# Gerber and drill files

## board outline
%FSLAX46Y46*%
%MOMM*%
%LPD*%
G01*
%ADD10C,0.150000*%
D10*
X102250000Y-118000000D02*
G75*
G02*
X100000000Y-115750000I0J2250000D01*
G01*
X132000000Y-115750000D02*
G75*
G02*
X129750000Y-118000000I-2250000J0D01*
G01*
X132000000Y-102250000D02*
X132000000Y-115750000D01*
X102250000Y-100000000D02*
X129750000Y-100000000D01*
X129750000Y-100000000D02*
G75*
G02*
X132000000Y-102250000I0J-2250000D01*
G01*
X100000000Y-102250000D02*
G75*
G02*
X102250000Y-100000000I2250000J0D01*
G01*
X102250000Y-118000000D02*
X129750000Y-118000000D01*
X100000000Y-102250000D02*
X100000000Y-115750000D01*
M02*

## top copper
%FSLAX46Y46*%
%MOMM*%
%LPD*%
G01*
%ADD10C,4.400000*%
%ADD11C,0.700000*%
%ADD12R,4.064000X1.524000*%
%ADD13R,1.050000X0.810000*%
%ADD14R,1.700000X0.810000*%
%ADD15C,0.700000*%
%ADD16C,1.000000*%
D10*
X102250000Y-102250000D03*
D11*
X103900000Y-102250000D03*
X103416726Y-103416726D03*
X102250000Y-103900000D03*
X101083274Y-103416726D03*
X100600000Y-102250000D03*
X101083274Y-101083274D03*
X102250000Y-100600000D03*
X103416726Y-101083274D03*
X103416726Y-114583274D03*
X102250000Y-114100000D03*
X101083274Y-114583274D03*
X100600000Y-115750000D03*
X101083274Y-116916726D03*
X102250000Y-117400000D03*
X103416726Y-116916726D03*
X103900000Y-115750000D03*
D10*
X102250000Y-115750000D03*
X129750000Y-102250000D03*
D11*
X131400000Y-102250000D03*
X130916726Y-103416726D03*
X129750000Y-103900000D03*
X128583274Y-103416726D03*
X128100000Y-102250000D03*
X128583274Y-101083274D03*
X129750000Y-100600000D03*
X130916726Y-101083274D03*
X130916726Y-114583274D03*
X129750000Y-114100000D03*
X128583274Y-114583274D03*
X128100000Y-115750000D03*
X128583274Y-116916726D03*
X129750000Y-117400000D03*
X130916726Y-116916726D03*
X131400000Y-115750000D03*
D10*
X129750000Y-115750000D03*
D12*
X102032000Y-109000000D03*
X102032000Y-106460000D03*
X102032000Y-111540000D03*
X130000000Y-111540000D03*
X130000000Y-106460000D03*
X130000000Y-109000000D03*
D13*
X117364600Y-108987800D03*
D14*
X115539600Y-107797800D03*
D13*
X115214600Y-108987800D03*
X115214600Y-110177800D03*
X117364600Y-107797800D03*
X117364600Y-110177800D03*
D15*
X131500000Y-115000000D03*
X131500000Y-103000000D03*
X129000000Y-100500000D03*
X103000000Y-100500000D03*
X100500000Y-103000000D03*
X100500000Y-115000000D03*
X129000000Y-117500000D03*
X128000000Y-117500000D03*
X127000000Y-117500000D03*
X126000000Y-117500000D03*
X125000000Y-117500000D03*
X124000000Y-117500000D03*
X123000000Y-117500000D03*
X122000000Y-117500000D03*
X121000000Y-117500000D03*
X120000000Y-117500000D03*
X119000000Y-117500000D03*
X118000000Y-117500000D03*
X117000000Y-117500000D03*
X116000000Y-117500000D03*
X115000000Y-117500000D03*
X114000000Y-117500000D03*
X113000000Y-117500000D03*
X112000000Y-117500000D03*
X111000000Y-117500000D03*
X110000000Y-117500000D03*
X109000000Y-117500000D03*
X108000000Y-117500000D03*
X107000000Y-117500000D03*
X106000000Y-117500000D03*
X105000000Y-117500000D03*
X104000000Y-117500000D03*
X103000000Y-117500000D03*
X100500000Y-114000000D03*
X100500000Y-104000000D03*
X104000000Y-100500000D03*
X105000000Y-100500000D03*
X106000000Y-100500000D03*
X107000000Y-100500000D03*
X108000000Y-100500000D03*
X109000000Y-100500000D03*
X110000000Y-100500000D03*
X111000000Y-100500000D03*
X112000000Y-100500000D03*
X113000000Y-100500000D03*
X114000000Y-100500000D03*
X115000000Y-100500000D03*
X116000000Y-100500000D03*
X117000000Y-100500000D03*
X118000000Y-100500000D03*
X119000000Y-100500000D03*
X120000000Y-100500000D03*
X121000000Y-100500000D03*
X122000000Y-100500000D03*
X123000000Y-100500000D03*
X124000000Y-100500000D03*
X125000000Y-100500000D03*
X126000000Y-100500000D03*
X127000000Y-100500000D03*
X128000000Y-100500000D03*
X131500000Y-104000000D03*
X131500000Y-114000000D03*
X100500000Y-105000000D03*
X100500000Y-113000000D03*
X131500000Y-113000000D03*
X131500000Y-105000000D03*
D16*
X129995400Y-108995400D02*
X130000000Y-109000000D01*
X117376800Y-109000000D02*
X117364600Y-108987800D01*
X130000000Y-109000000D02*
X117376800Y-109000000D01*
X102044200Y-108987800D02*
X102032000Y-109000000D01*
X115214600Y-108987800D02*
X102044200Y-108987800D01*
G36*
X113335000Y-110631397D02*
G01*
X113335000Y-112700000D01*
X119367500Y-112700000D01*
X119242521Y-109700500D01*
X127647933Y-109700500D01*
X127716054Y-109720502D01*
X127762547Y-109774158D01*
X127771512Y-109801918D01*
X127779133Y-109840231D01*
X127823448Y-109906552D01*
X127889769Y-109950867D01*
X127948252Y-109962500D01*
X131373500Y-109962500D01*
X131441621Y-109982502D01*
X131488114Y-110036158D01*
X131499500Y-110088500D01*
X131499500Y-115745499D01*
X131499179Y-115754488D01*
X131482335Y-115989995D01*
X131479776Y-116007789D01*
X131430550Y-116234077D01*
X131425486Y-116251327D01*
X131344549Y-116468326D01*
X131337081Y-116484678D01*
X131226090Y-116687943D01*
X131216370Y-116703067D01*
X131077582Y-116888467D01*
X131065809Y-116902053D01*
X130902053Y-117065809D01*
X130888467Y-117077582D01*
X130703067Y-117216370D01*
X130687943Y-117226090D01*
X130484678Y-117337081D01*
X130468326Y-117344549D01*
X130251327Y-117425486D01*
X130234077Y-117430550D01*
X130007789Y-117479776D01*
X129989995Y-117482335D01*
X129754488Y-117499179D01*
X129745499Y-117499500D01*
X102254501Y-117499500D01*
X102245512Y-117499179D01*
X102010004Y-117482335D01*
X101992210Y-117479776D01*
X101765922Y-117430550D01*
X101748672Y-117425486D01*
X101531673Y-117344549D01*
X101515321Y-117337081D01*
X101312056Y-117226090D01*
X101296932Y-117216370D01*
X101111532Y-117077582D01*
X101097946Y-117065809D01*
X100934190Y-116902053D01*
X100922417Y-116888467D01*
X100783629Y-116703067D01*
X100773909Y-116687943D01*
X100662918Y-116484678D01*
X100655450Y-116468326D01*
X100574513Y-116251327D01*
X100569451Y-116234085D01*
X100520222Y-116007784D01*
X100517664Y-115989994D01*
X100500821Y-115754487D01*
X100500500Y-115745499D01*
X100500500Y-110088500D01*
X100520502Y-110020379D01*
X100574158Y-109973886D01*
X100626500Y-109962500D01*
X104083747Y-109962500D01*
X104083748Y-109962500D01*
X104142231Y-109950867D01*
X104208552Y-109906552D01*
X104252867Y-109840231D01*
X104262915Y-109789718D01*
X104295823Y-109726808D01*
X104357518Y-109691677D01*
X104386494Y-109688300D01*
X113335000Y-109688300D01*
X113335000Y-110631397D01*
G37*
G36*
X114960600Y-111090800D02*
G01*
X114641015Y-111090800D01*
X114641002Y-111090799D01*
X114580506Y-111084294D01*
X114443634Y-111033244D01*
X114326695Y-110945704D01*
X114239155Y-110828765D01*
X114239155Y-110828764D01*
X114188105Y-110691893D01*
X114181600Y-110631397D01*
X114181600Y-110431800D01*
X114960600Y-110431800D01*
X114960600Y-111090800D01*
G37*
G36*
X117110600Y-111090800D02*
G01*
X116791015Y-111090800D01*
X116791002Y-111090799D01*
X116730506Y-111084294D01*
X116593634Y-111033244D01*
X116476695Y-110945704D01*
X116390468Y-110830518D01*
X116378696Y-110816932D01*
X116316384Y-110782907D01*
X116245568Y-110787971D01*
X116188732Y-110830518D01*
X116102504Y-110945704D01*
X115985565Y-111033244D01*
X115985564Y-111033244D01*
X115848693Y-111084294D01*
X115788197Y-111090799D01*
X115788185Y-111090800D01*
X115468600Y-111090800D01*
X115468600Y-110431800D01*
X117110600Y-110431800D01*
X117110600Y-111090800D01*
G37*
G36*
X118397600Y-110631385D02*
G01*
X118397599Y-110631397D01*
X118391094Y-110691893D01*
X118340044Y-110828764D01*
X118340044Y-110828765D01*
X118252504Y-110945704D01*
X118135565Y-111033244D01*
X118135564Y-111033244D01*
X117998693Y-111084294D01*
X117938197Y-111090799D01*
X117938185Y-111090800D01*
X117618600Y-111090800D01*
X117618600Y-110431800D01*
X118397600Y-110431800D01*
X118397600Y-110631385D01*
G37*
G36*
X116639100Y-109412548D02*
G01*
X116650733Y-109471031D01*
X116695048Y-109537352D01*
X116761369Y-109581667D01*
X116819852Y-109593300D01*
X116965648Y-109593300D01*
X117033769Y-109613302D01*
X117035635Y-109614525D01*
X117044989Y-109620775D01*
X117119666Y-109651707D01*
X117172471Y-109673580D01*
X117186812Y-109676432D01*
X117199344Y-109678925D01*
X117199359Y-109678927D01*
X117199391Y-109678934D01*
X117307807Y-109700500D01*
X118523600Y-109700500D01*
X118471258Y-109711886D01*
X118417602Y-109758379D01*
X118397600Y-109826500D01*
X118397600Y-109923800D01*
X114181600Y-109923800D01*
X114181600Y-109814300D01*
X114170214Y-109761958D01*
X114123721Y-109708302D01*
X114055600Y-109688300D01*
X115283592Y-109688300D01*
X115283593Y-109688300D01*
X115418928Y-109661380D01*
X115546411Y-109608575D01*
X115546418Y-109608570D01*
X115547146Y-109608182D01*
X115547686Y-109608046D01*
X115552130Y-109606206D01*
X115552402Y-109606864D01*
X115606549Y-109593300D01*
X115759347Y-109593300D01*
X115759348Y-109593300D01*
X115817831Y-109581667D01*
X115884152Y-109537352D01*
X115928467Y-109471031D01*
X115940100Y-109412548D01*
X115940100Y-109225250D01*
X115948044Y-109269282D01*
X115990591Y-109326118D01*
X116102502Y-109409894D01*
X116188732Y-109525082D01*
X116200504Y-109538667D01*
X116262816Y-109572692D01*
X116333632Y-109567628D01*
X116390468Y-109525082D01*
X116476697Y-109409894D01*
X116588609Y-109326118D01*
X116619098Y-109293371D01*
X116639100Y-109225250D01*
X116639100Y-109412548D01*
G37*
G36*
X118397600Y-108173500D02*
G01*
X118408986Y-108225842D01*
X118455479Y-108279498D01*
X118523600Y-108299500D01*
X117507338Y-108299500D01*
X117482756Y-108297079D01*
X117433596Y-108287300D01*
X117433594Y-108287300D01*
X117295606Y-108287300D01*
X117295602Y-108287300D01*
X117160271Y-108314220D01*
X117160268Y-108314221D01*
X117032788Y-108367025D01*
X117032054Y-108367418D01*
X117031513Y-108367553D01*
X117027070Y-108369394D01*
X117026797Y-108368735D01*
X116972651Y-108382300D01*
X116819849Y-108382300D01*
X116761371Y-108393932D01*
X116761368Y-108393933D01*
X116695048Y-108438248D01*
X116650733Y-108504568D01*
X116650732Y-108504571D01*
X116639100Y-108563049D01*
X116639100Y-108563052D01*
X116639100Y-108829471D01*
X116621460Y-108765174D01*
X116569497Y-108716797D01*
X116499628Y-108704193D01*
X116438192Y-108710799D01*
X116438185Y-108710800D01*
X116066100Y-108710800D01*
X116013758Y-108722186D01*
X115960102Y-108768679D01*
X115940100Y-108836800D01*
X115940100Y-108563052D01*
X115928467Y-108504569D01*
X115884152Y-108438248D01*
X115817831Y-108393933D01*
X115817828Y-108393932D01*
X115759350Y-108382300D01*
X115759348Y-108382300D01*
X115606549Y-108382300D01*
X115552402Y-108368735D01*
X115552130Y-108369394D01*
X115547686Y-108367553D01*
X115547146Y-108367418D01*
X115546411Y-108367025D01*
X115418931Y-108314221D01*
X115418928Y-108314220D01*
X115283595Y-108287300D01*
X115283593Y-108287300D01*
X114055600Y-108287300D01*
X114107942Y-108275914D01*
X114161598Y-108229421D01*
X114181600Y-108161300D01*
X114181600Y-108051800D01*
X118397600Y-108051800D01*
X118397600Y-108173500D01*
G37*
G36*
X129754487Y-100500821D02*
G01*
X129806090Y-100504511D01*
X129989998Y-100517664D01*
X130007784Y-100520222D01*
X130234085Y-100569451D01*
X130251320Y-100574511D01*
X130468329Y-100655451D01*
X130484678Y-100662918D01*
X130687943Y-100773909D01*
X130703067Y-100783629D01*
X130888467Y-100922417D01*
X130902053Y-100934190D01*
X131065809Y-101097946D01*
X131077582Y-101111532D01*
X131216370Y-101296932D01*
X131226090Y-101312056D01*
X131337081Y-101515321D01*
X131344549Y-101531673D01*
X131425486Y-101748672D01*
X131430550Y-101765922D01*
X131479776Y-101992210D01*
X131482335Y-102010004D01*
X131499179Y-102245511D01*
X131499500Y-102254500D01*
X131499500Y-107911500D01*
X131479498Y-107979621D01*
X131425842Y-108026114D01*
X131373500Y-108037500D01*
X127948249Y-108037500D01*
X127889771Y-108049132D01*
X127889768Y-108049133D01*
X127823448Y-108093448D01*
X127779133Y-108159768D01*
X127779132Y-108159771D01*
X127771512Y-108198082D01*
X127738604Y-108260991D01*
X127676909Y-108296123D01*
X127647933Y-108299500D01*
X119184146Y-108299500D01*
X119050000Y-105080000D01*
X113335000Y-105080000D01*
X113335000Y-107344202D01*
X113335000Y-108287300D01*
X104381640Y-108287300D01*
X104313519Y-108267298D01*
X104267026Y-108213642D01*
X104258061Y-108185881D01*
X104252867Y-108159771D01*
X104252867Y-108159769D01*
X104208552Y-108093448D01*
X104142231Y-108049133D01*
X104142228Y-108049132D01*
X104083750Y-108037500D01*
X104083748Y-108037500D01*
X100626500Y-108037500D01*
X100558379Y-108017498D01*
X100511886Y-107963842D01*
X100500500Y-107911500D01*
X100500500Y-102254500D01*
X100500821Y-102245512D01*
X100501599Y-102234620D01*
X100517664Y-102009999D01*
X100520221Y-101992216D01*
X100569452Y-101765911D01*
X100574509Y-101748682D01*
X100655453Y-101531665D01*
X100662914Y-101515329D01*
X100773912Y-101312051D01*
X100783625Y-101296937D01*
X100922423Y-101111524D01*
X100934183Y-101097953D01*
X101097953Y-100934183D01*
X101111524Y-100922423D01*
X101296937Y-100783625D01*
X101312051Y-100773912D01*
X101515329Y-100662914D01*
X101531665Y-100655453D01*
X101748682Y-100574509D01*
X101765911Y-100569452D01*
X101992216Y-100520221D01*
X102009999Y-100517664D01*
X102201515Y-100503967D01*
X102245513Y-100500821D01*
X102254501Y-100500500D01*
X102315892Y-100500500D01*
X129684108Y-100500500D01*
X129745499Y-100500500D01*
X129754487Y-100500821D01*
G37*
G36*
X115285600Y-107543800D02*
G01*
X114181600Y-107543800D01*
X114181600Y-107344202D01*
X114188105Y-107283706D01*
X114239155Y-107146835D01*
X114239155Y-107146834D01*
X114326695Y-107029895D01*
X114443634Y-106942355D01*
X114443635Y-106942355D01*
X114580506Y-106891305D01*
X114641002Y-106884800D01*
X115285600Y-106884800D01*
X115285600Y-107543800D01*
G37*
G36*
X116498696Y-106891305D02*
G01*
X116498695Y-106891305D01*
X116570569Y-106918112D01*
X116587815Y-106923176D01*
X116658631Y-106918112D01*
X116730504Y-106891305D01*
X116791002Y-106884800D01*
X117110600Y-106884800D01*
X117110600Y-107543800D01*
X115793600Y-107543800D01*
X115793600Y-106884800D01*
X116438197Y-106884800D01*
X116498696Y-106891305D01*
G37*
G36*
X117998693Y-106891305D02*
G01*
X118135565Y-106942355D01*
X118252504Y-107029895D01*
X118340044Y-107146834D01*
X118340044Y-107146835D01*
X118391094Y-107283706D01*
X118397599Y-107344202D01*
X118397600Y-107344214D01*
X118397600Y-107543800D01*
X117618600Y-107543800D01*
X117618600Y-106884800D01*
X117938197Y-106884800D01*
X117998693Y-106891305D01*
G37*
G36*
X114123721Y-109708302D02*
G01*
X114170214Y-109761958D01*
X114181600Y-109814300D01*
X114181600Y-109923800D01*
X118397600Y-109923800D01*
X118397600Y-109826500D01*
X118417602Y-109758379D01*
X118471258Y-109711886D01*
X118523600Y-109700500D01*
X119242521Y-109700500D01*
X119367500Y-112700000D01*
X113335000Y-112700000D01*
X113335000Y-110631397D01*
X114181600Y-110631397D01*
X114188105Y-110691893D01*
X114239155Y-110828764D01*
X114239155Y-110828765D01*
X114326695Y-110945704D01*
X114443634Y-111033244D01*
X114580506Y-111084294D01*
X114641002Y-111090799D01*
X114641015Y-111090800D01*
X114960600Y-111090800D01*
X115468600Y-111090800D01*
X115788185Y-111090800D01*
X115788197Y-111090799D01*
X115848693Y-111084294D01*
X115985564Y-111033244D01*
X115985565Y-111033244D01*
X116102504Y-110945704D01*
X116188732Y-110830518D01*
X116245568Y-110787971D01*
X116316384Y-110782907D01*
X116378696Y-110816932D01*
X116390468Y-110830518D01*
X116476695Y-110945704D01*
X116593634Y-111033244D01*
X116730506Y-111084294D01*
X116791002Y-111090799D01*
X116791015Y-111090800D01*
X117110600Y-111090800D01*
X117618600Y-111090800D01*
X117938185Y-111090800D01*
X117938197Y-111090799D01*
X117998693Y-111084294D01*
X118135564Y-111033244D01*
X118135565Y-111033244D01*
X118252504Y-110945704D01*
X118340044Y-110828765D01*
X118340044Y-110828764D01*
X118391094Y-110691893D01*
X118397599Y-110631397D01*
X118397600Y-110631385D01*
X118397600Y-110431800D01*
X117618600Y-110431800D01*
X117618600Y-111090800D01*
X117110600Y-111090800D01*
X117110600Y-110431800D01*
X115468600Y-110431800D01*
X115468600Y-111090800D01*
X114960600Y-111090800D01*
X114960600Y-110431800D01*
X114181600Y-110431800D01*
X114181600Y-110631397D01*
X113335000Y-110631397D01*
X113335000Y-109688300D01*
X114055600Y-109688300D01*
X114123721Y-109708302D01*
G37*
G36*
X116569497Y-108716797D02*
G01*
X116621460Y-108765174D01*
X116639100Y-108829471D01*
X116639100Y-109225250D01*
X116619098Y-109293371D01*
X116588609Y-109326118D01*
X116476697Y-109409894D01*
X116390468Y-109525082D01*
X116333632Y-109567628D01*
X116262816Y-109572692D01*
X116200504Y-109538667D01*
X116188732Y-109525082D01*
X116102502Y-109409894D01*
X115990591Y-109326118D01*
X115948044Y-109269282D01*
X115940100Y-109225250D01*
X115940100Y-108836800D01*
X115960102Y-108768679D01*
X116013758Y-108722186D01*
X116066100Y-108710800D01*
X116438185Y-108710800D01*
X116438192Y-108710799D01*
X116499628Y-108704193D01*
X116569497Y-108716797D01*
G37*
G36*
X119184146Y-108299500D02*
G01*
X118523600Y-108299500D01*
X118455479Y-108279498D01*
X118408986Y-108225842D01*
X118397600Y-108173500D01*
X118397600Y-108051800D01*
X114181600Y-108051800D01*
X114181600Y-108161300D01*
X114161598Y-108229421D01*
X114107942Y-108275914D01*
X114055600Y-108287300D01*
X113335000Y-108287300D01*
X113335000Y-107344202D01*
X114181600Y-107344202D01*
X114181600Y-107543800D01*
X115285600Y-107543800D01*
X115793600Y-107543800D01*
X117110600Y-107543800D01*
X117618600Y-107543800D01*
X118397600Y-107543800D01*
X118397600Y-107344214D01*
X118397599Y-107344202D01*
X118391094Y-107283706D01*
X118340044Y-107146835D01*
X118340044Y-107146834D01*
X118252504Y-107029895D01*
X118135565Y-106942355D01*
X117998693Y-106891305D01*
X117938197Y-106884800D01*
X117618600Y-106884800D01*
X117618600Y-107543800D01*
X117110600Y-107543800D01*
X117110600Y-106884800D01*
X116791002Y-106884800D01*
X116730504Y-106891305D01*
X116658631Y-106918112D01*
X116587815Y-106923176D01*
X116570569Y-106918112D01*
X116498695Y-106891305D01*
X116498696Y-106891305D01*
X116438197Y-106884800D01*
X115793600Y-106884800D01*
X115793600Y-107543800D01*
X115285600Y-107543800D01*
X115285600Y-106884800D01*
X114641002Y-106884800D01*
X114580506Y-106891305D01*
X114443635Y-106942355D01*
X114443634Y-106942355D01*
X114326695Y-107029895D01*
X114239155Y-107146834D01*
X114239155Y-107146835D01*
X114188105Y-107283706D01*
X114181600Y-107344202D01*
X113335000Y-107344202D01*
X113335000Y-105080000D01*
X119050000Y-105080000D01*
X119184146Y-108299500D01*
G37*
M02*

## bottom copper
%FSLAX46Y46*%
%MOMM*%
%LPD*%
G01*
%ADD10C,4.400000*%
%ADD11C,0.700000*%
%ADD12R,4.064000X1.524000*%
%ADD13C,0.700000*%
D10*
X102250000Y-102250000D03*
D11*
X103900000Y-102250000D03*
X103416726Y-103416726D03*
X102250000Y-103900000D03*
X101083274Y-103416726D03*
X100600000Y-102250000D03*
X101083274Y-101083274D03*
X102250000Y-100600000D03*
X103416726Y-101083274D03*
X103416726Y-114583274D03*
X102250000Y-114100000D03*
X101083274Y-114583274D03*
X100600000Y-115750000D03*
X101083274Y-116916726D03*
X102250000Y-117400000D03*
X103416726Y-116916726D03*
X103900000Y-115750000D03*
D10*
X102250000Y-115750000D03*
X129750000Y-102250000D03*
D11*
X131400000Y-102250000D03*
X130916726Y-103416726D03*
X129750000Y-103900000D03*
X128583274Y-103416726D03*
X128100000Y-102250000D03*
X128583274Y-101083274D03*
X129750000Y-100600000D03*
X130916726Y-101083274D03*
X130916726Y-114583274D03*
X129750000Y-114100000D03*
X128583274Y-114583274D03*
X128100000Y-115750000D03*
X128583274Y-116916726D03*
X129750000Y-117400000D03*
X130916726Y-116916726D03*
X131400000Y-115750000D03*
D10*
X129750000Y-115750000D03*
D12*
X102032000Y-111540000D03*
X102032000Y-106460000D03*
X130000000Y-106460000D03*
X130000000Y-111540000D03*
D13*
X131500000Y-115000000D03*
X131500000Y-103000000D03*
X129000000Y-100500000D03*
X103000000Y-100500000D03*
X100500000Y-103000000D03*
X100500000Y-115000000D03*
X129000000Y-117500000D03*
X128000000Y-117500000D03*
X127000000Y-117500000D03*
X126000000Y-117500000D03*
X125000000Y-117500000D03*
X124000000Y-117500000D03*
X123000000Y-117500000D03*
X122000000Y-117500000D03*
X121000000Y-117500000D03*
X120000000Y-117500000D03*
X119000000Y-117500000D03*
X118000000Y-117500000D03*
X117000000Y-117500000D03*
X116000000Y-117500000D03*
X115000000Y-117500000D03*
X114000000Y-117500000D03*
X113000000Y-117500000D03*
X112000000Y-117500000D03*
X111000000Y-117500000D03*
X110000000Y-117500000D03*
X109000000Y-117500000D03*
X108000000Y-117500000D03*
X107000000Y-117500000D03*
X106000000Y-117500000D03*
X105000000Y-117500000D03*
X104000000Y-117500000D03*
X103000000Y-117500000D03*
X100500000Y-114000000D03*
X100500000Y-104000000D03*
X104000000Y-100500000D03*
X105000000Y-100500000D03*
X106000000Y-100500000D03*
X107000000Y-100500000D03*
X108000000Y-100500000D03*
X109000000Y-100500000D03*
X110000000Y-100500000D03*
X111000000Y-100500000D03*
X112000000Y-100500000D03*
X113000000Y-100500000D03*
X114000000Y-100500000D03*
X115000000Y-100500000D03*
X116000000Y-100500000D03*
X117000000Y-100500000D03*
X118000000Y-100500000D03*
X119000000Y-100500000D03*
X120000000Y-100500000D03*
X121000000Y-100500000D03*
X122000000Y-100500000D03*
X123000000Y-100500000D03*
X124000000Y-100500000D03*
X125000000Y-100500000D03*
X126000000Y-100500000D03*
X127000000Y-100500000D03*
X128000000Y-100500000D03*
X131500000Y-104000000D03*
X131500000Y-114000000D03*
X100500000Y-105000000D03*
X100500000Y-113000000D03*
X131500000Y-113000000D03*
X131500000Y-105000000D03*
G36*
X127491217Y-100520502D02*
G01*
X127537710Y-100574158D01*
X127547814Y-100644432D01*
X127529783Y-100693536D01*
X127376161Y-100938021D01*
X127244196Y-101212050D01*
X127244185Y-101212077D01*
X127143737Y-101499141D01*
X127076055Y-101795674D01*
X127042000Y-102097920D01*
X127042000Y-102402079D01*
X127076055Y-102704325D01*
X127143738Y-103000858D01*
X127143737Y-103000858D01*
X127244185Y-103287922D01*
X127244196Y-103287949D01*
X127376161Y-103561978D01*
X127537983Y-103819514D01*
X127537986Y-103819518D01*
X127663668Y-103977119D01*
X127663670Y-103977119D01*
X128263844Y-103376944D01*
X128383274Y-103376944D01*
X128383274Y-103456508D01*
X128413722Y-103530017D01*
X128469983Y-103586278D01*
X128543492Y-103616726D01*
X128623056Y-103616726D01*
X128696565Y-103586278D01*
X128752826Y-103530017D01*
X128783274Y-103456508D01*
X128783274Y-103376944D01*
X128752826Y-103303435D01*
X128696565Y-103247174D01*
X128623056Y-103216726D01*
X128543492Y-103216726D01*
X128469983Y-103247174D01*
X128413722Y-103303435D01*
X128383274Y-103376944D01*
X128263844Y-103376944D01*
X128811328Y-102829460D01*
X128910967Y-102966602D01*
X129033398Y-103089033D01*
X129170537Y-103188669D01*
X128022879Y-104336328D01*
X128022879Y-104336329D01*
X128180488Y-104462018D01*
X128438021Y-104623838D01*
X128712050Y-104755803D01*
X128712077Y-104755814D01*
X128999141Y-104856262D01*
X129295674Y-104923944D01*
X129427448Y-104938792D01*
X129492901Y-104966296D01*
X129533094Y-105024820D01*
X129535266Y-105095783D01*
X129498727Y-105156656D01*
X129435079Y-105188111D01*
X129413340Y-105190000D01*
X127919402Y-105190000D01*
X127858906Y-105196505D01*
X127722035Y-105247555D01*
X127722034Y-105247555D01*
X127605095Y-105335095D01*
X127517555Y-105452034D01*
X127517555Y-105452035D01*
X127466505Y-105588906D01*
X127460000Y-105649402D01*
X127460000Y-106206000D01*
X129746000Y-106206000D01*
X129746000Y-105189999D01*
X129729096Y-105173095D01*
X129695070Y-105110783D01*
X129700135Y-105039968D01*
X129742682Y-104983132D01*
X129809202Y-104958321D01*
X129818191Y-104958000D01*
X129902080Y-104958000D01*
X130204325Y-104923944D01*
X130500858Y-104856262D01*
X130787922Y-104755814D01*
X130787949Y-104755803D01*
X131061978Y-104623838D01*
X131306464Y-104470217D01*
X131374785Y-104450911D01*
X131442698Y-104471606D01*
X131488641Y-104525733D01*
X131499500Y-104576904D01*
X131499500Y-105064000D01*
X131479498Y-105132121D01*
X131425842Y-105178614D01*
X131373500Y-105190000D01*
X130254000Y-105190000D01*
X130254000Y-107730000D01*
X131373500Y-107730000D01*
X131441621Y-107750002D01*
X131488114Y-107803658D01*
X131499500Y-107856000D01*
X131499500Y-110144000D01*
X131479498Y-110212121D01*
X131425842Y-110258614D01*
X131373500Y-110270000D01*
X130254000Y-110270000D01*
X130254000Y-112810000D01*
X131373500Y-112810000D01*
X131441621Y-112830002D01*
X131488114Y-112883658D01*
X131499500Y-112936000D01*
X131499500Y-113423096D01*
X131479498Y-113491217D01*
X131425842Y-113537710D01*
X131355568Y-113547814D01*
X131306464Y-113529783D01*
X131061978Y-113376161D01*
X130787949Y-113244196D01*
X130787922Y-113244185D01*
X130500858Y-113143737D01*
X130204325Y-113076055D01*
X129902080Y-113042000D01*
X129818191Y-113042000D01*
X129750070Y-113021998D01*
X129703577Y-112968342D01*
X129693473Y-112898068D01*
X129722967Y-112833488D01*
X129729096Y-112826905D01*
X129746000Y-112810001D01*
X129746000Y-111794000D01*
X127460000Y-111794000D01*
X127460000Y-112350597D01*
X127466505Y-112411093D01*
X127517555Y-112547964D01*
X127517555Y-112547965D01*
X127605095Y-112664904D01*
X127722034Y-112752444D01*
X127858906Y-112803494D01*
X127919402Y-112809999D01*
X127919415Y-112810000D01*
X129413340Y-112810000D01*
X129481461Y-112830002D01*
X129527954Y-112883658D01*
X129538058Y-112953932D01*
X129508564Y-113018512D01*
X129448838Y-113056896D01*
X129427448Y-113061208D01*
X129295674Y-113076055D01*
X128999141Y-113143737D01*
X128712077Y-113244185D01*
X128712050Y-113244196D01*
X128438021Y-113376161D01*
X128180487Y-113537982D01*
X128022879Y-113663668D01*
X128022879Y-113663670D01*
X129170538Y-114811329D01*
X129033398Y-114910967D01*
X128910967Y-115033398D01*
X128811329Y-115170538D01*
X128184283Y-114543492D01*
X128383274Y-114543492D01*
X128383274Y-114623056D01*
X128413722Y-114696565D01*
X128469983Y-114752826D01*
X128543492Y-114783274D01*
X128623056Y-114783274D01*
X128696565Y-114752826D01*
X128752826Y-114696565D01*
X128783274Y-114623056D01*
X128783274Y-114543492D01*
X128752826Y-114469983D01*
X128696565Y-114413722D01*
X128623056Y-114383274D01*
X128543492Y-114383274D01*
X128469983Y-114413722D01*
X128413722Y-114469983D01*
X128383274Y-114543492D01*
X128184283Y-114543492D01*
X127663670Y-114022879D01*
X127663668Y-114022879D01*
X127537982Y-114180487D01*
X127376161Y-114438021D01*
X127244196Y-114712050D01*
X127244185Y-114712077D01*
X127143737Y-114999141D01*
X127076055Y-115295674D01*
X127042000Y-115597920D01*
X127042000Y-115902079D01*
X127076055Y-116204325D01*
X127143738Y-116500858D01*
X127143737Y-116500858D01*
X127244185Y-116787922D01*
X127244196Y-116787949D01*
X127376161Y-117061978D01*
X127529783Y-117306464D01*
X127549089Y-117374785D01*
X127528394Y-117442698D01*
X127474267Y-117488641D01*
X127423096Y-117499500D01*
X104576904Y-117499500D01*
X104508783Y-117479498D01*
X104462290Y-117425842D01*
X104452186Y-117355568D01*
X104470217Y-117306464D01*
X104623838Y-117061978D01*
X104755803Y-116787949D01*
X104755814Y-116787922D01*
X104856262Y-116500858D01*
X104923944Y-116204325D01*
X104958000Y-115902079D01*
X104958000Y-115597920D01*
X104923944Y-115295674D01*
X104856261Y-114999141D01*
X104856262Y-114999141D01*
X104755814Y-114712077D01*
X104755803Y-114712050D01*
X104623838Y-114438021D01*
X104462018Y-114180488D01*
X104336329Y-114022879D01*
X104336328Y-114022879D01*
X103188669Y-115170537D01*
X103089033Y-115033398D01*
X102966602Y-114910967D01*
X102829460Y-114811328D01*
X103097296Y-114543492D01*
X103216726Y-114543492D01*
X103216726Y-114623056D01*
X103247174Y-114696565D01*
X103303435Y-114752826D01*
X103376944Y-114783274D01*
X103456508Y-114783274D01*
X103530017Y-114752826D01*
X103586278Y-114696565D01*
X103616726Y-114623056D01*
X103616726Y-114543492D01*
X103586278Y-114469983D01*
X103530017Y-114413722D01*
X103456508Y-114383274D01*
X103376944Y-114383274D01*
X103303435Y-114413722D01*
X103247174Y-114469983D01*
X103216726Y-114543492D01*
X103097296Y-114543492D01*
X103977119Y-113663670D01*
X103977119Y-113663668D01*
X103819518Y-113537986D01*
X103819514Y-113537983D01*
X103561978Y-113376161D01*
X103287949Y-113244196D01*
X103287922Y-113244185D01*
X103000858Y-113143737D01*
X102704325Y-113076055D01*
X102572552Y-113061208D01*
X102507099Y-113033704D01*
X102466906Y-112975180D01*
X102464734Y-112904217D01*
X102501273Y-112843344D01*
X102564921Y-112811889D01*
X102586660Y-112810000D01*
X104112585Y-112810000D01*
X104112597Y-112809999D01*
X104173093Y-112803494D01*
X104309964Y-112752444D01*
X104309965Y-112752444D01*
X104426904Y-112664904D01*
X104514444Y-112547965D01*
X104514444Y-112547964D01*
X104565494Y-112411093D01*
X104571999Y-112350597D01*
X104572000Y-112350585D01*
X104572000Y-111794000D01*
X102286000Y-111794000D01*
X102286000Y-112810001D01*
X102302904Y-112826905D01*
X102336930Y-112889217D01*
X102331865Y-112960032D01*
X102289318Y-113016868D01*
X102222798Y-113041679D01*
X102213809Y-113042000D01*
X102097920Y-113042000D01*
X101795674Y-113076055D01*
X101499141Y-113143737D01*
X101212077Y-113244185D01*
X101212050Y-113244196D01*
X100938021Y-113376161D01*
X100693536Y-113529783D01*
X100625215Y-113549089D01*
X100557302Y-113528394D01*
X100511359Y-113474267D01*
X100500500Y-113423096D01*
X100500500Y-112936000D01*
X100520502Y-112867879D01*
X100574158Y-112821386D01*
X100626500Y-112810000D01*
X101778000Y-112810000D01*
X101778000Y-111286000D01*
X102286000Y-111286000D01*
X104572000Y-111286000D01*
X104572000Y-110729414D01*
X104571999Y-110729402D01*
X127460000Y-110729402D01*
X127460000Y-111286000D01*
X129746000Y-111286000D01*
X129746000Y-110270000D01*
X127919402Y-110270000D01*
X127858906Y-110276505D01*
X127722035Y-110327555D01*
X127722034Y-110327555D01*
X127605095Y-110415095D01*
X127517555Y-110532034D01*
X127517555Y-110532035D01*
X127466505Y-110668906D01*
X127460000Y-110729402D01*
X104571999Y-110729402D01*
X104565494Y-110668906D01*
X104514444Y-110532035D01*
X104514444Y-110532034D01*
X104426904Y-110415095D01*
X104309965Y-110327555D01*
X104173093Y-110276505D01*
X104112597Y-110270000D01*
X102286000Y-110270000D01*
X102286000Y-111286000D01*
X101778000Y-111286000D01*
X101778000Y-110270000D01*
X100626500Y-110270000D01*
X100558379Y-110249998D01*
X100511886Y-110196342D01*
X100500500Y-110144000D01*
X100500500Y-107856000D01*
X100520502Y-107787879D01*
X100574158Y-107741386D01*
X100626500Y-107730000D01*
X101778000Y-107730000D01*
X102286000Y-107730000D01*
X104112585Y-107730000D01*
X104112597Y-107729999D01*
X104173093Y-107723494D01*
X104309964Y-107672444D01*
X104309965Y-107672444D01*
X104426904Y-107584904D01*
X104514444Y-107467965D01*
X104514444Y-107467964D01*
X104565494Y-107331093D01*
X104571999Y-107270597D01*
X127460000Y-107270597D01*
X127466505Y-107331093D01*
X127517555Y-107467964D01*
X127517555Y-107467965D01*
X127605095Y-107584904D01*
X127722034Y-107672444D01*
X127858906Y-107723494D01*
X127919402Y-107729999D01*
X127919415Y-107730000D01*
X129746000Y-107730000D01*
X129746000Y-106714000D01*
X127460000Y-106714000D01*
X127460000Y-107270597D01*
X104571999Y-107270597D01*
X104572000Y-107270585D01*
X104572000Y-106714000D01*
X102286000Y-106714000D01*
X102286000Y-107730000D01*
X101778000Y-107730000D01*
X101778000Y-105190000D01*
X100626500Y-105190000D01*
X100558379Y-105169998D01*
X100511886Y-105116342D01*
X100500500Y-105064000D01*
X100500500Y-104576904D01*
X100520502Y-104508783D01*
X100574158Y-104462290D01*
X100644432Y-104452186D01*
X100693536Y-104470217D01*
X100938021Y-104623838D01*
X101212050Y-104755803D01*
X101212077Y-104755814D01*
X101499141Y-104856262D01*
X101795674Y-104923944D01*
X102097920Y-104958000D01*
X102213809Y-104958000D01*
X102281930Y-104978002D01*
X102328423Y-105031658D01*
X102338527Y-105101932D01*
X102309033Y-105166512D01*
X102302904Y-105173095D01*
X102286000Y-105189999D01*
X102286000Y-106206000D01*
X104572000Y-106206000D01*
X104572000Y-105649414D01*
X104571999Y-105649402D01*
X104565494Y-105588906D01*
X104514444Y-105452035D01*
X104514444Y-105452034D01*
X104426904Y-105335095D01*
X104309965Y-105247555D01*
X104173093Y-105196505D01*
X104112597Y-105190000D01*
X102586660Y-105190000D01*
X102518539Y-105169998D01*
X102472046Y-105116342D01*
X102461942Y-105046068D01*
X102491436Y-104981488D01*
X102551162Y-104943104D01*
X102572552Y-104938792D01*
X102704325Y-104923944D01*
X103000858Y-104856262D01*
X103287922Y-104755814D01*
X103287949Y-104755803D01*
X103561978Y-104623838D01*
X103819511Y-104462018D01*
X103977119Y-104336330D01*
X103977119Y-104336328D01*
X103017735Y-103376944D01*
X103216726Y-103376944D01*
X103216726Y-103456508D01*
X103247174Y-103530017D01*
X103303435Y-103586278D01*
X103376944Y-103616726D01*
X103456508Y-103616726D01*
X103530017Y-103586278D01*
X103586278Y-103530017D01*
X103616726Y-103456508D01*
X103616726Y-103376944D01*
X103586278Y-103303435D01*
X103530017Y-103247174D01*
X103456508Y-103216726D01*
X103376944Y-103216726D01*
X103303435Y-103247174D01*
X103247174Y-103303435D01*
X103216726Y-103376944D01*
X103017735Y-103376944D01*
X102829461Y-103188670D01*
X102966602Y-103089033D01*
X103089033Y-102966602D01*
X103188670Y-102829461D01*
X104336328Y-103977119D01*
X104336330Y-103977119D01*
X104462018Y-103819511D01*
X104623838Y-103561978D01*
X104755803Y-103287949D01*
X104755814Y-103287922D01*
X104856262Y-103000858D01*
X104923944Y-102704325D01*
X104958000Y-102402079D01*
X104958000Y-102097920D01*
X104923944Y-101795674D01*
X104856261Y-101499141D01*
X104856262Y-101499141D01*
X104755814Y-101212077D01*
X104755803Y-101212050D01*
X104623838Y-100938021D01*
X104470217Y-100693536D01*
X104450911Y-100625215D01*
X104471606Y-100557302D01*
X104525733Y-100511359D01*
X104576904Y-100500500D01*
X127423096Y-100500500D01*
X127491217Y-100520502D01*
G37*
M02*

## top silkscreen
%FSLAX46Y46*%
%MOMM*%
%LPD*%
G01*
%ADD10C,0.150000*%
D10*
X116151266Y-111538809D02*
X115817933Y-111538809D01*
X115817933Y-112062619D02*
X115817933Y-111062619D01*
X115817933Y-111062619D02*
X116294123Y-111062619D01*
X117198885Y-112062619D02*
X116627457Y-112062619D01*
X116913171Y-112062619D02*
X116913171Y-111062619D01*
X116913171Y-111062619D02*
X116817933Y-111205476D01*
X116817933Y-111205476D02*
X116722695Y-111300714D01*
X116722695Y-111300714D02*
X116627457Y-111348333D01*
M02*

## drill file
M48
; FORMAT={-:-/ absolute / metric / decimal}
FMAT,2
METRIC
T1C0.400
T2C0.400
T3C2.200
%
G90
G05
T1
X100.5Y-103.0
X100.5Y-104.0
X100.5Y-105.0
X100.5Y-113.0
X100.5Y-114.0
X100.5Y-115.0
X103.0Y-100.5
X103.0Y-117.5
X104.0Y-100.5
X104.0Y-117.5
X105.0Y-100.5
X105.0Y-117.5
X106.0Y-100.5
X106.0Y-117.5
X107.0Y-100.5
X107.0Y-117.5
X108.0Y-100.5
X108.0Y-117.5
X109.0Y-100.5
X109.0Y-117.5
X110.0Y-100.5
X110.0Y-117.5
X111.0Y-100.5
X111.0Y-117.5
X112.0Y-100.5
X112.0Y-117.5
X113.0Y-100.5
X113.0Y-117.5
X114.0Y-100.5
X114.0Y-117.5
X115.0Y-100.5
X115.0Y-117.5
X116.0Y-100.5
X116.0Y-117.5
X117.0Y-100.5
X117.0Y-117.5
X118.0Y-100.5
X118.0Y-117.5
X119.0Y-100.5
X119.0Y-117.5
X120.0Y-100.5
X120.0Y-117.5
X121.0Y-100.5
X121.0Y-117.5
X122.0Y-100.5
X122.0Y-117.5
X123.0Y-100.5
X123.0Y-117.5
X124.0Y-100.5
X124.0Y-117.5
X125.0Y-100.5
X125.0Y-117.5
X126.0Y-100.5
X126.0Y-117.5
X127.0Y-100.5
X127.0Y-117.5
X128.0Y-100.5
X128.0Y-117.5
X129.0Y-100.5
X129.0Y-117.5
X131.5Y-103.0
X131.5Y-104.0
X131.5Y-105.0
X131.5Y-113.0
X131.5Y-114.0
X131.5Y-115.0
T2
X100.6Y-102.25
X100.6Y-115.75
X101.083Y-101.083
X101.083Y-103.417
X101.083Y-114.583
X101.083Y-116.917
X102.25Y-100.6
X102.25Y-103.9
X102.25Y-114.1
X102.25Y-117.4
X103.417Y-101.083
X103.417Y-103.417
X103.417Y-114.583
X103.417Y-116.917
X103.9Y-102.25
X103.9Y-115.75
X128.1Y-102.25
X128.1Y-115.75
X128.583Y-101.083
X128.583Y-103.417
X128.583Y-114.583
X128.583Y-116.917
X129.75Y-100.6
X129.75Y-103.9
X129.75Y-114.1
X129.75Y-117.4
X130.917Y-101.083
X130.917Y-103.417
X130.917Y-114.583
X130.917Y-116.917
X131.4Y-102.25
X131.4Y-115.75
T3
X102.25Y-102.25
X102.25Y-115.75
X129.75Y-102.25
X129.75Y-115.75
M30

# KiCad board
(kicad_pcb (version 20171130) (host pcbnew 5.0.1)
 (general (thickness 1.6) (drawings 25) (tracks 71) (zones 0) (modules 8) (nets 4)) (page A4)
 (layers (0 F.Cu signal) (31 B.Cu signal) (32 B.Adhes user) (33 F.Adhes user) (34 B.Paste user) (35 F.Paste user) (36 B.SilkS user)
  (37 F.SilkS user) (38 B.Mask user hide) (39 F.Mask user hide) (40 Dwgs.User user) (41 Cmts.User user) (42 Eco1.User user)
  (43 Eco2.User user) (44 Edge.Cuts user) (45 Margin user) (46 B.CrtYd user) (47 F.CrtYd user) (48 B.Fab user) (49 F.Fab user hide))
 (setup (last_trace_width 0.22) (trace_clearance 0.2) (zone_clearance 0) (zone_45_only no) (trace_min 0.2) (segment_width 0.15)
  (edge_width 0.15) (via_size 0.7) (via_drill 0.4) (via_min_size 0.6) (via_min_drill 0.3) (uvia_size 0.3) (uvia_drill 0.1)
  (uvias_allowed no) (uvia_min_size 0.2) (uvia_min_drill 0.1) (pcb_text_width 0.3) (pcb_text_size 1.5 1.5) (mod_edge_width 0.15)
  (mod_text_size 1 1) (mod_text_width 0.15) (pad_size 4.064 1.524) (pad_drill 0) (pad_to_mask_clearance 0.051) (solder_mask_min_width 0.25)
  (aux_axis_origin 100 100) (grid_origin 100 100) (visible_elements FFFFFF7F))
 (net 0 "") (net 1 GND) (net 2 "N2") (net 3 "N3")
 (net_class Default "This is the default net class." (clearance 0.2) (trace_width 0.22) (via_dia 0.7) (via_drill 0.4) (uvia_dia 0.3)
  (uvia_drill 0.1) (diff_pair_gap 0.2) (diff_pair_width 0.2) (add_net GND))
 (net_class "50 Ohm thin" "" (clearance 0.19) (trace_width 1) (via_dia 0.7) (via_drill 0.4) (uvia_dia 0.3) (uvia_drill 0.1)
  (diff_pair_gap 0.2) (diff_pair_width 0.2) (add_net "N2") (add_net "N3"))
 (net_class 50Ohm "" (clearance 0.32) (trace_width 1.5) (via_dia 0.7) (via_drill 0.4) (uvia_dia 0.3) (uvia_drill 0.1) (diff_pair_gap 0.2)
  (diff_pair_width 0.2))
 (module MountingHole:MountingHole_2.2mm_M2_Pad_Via (layer F.Cu) (at 102.25 102.25)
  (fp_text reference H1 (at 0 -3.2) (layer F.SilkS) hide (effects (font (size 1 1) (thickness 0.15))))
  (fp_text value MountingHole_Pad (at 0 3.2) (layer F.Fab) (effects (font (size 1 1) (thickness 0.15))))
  (pad 1 thru_hole circle (at 0 0) (size 4.4 4.4) (drill 2.2) (layers *.Cu *.Mask) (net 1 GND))
  (pad 1 thru_hole circle (at 1.65 0) (size 0.7 0.7) (drill 0.4) (layers *.Cu *.Mask) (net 1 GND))
  (pad 1 thru_hole circle (at 1.166726 1.166726) (size 0.7 0.7) (drill 0.4) (layers *.Cu *.Mask) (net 1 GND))
  (pad 1 thru_hole circle (at 0 1.65) (size 0.7 0.7) (drill 0.4) (layers *.Cu *.Mask) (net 1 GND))
  (pad 1 thru_hole circle (at -1.166726 1.166726) (size 0.7 0.7) (drill 0.4) (layers *.Cu *.Mask) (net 1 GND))
  (pad 1 thru_hole circle (at -1.65 0) (size 0.7 0.7) (drill 0.4) (layers *.Cu *.Mask) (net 1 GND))
  (pad 1 thru_hole circle (at -1.166726 -1.166726) (size 0.7 0.7) (drill 0.4) (layers *.Cu *.Mask) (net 1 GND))
  (pad 1 thru_hole circle (at 0 -1.65) (size 0.7 0.7) (drill 0.4) (layers *.Cu *.Mask) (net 1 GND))
  (pad 1 thru_hole circle (at 1.166726 -1.166726) (size 0.7 0.7) (drill 0.4) (layers *.Cu *.Mask) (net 1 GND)))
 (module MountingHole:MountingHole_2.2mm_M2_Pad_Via (layer F.Cu) (at 102.25 115.75)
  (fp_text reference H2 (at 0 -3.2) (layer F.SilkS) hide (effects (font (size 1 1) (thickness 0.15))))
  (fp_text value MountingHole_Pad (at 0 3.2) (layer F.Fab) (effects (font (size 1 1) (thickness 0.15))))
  (pad 1 thru_hole circle (at 1.166726 -1.166726) (size 0.7 0.7) (drill 0.4) (layers *.Cu *.Mask) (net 1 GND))
  (pad 1 thru_hole circle (at 0 -1.65) (size 0.7 0.7) (drill 0.4) (layers *.Cu *.Mask) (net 1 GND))
  (pad 1 thru_hole circle (at -1.166726 -1.166726) (size 0.7 0.7) (drill 0.4) (layers *.Cu *.Mask) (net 1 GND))
  (pad 1 thru_hole circle (at -1.65 0) (size 0.7 0.7) (drill 0.4) (layers *.Cu *.Mask) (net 1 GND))
  (pad 1 thru_hole circle (at -1.166726 1.166726) (size 0.7 0.7) (drill 0.4) (layers *.Cu *.Mask) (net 1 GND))
  (pad 1 thru_hole circle (at 0 1.65) (size 0.7 0.7) (drill 0.4) (layers *.Cu *.Mask) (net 1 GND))
  (pad 1 thru_hole circle (at 1.166726 1.166726) (size 0.7 0.7) (drill 0.4) (layers *.Cu *.Mask) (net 1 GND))
  (pad 1 thru_hole circle (at 1.65 0) (size 0.7 0.7) (drill 0.4) (layers *.Cu *.Mask) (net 1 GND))
  (pad 1 thru_hole circle (at 0 0) (size 4.4 4.4) (drill 2.2) (layers *.Cu *.Mask) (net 1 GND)))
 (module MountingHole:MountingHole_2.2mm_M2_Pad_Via (layer F.Cu) (at 129.75 102.25)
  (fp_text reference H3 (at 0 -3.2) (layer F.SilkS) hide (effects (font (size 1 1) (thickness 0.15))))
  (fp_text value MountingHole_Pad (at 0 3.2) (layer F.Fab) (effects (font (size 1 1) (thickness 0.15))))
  (pad 1 thru_hole circle (at 0 0) (size 4.4 4.4) (drill 2.2) (layers *.Cu *.Mask) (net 1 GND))
  (pad 1 thru_hole circle (at 1.65 0) (size 0.7 0.7) (drill 0.4) (layers *.Cu *.Mask) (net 1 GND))
  (pad 1 thru_hole circle (at 1.166726 1.166726) (size 0.7 0.7) (drill 0.4) (layers *.Cu *.Mask) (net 1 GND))
  (pad 1 thru_hole circle (at 0 1.65) (size 0.7 0.7) (drill 0.4) (layers *.Cu *.Mask) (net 1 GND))
  (pad 1 thru_hole circle (at -1.166726 1.166726) (size 0.7 0.7) (drill 0.4) (layers *.Cu *.Mask) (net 1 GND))
  (pad 1 thru_hole circle (at -1.65 0) (size 0.7 0.7) (drill 0.4) (layers *.Cu *.Mask) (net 1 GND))
  (pad 1 thru_hole circle (at -1.166726 -1.166726) (size 0.7 0.7) (drill 0.4) (layers *.Cu *.Mask) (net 1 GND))
  (pad 1 thru_hole circle (at 0 -1.65) (size 0.7 0.7) (drill 0.4) (layers *.Cu *.Mask) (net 1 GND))
  (pad 1 thru_hole circle (at 1.166726 -1.166726) (size 0.7 0.7) (drill 0.4) (layers *.Cu *.Mask) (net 1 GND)))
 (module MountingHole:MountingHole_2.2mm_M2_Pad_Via (layer F.Cu) (at 129.75 115.75)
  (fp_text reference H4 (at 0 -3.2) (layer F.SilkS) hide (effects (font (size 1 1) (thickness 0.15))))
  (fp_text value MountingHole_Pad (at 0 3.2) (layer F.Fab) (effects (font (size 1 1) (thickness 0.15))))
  (pad 1 thru_hole circle (at 1.166726 -1.166726) (size 0.7 0.7) (drill 0.4) (layers *.Cu *.Mask) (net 1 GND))
  (pad 1 thru_hole circle (at 0 -1.65) (size 0.7 0.7) (drill 0.4) (layers *.Cu *.Mask) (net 1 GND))
  (pad 1 thru_hole circle (at -1.166726 -1.166726) (size 0.7 0.7) (drill 0.4) (layers *.Cu *.Mask) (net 1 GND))
  (pad 1 thru_hole circle (at -1.65 0) (size 0.7 0.7) (drill 0.4) (layers *.Cu *.Mask) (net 1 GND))
  (pad 1 thru_hole circle (at -1.166726 1.166726) (size 0.7 0.7) (drill 0.4) (layers *.Cu *.Mask) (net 1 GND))
  (pad 1 thru_hole circle (at 0 1.65) (size 0.7 0.7) (drill 0.4) (layers *.Cu *.Mask) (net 1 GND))
  (pad 1 thru_hole circle (at 1.166726 1.166726) (size 0.7 0.7) (drill 0.4) (layers *.Cu *.Mask) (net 1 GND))
  (pad 1 thru_hole circle (at 1.65 0) (size 0.7 0.7) (drill 0.4) (layers *.Cu *.Mask) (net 1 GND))
  (pad 1 thru_hole circle (at 0 0) (size 4.4 4.4) (drill 2.2) (layers *.Cu *.Mask) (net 1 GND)))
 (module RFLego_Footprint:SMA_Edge (layer F.Cu) (at 100 109)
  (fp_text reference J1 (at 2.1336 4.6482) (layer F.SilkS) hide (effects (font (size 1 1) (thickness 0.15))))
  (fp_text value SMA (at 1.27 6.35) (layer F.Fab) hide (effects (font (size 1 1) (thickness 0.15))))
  (pad 1 smd rect (at 2.032 0) (size 4.064 1.524) (layers F.Cu F.Mask) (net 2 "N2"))
  (pad 2 smd rect (at 2.032 -2.54) (size 4.064 1.524) (layers F.Cu F.Mask) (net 1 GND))
  (pad 2 smd rect (at 2.032 2.54) (size 4.064 1.524) (layers B.Cu B.Mask) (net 1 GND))
  (pad 2 smd rect (at 2.032 -2.54) (size 4.064 1.524) (layers B.Cu B.Mask) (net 1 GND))
  (pad 2 smd rect (at 2.032 2.54) (size 4.064 1.524) (layers F.Cu F.Mask) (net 1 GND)))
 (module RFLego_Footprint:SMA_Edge (layer F.Cu) (at 127.968 109)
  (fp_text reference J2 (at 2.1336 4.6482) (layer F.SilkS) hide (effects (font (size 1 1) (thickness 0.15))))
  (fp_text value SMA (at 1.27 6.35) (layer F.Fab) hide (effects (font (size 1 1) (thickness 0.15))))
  (pad 2 smd rect (at 2.032 2.54) (size 4.064 1.524) (layers F.Cu F.Mask) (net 1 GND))
  (pad 2 smd rect (at 2.032 -2.54) (size 4.064 1.524) (layers B.Cu B.Mask) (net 1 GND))
  (pad 2 smd rect (at 2.032 2.54) (size 4.064 1.524) (layers B.Cu B.Mask) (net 1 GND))
  (pad 2 smd rect (at 2.032 -2.54) (size 4.064 1.524) (layers F.Cu F.Mask) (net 1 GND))
  (pad 1 smd rect (at 2.032 0) (size 4.064 1.524) (layers F.Cu F.Mask) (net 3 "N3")))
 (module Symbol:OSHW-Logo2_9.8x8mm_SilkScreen (layer B.Cu) (at 109.5 113.25 180)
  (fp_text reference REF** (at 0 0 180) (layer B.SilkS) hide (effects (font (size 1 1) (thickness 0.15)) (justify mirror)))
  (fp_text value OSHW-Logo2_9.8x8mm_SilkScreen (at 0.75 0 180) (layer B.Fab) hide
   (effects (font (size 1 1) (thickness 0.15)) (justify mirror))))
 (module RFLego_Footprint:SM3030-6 (layer F.Cu) (at 115.2146 107.7978)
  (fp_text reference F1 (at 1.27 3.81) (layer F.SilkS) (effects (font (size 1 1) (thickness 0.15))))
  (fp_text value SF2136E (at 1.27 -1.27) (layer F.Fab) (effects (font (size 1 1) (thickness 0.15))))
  (pad 2 smd rect (at 2.15 1.19) (size 1.05 0.81) (layers F.Cu F.Paste F.Mask) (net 3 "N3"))
  (pad 3 smd rect (at 0.325 0) (size 1.7 0.81) (layers F.Cu F.Paste F.Mask) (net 1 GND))
  (pad 1 smd rect (at 0 1.19) (size 1.05 0.81) (layers F.Cu F.Paste F.Mask) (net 2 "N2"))
  (pad 3 smd rect (at 0 2.38) (size 1.05 0.81) (layers F.Cu F.Paste F.Mask) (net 1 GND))
  (pad 3 smd rect (at 2.15 0) (size 1.05 0.81) (layers F.Cu F.Paste F.Mask) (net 1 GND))
  (pad 3 smd rect (at 2.15 2.38) (size 1.05 0.81) (layers F.Cu F.Paste F.Mask) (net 1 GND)))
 (gr_arc (start 102.25 115.75) (end 100 115.75) (angle -90) (layer Edge.Cuts) (width 0.15))
 (gr_arc (start 129.75 115.75) (end 129.75 118) (angle -90) (layer Edge.Cuts) (width 0.15))
 (gr_line (start 132 102.25) (end 132 115.75) (layer Edge.Cuts) (width 0.15))
 (gr_line (start 102.25 100) (end 129.75 100) (layer Edge.Cuts) (width 0.15))
 (gr_arc (start 129.75 102.25) (end 132 102.25) (angle -90) (layer Edge.Cuts) (width 0.15))
 (gr_arc (start 102.25 102.25) (end 102.25 100) (angle -90) (layer Edge.Cuts) (width 0.15))
 (gr_line (start 102.25 118) (end 129.75 118) (layer Edge.Cuts) (width 0.15))
 (gr_line (start 100 102.25) (end 100 115.75) (layer Edge.Cuts) (width 0.15))
 (via (at 131.5 115) (size 0.7) (drill 0.4) (layers F.Cu B.Cu) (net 1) (status 30))
 (via (at 131.5 103) (size 0.7) (drill 0.4) (layers F.Cu B.Cu) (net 1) (status 30))
 (via (at 129 100.5) (size 0.7) (drill 0.4) (layers F.Cu B.Cu) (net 1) (status 30))
 (via (at 103 100.5) (size 0.7) (drill 0.4) (layers F.Cu B.Cu) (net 1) (status 30))
 (via (at 100.5 103) (size 0.7) (drill 0.4) (layers F.Cu B.Cu) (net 1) (status 30))
 (via (at 100.5 115) (size 0.7) (drill 0.4) (layers F.Cu B.Cu) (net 1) (status 30))
 (via (at 129 117.5) (size 0.7) (drill 0.4) (layers F.Cu B.Cu) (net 1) (status 30))
 (via (at 128 117.5) (size 0.7) (drill 0.4) (layers F.Cu B.Cu) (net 1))
 (via (at 127 117.5) (size 0.7) (drill 0.4) (layers F.Cu B.Cu) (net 1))
 (via (at 126 117.5) (size 0.7) (drill 0.4) (layers F.Cu B.Cu) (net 1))
 (via (at 125 117.5) (size 0.7) (drill 0.4) (layers F.Cu B.Cu) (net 1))
 (via (at 124 117.5) (size 0.7) (drill 0.4) (layers F.Cu B.Cu) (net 1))
 (via (at 123 117.5) (size 0.7) (drill 0.4) (layers F.Cu B.Cu) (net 1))
 (via (at 122 117.5) (size 0.7) (drill 0.4) (layers F.Cu B.Cu) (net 1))
 (via (at 121 117.5) (size 0.7) (drill 0.4) (layers F.Cu B.Cu) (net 1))
 (via (at 120 117.5) (size 0.7) (drill 0.4) (layers F.Cu B.Cu) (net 1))
 (via (at 119 117.5) (size 0.7) (drill 0.4) (layers F.Cu B.Cu) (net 1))
 (via (at 118 117.5) (size 0.7) (drill 0.4) (layers F.Cu B.Cu) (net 1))
 (via (at 117 117.5) (size 0.7) (drill 0.4) (layers F.Cu B.Cu) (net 1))
 (via (at 116 117.5) (size 0.7) (drill 0.4) (layers F.Cu B.Cu) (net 1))
 (via (at 115 117.5) (size 0.7) (drill 0.4) (layers F.Cu B.Cu) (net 1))
 (via (at 114 117.5) (size 0.7) (drill 0.4) (layers F.Cu B.Cu) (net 1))
 (via (at 113 117.5) (size 0.7) (drill 0.4) (layers F.Cu B.Cu) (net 1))
 (via (at 112 117.5) (size 0.7) (drill 0.4) (layers F.Cu B.Cu) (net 1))
 (via (at 111 117.5) (size 0.7) (drill 0.4) (layers F.Cu B.Cu) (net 1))
 (via (at 110 117.5) (size 0.7) (drill 0.4) (layers F.Cu B.Cu) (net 1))
 (via (at 109 117.5) (size 0.7) (drill 0.4) (layers F.Cu B.Cu) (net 1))
 (via (at 108 117.5) (size 0.7) (drill 0.4) (layers F.Cu B.Cu) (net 1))
 (via (at 107 117.5) (size 0.7) (drill 0.4) (layers F.Cu B.Cu) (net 1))
 (via (at 106 117.5) (size 0.7) (drill 0.4) (layers F.Cu B.Cu) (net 1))
 (via (at 105 117.5) (size 0.7) (drill 0.4) (layers F.Cu B.Cu) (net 1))
 (via (at 104 117.5) (size 0.7) (drill 0.4) (layers F.Cu B.Cu) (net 1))
 (via (at 103 117.5) (size 0.7) (drill 0.4) (layers F.Cu B.Cu) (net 1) (status 30))
 (via (at 100.5 114) (size 0.7) (drill 0.4) (layers F.Cu B.Cu) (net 1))
 (via (at 100.5 104) (size 0.7) (drill 0.4) (layers F.Cu B.Cu) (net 1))
 (via (at 104 100.5) (size 0.7) (drill 0.4) (layers F.Cu B.Cu) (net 1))
 (via (at 105 100.5) (size 0.7) (drill 0.4) (layers F.Cu B.Cu) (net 1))
 (via (at 106 100.5) (size 0.7) (drill 0.4) (layers F.Cu B.Cu) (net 1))
 (via (at 107 100.5) (size 0.7) (drill 0.4) (layers F.Cu B.Cu) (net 1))
 (via (at 108 100.5) (size 0.7) (drill 0.4) (layers F.Cu B.Cu) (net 1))
 (via (at 109 100.5) (size 0.7) (drill 0.4) (layers F.Cu B.Cu) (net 1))
 (via (at 110 100.5) (size 0.7) (drill 0.4) (layers F.Cu B.Cu) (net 1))
 (via (at 111 100.5) (size 0.7) (drill 0.4) (layers F.Cu B.Cu) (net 1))
 (via (at 112 100.5) (size 0.7) (drill 0.4) (layers F.Cu B.Cu) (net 1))
 (via (at 113 100.5) (size 0.7) (drill 0.4) (layers F.Cu B.Cu) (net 1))
 (via (at 114 100.5) (size 0.7) (drill 0.4) (layers F.Cu B.Cu) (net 1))
 (via (at 115 100.5) (size 0.7) (drill 0.4) (layers F.Cu B.Cu) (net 1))
 (via (at 116 100.5) (size 0.7) (drill 0.4) (layers F.Cu B.Cu) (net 1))
 (via (at 117 100.5) (size 0.7) (drill 0.4) (layers F.Cu B.Cu) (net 1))
 (via (at 118 100.5) (size 0.7) (drill 0.4) (layers F.Cu B.Cu) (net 1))
 (via (at 119 100.5) (size 0.7) (drill 0.4) (layers F.Cu B.Cu) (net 1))
 (via (at 120 100.5) (size 0.7) (drill 0.4) (layers F.Cu B.Cu) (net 1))
 (via (at 121 100.5) (size 0.7) (drill 0.4) (layers F.Cu B.Cu) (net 1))
 (via (at 122 100.5) (size 0.7) (drill 0.4) (layers F.Cu B.Cu) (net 1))
 (via (at 123 100.5) (size 0.7) (drill 0.4) (layers F.Cu B.Cu) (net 1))
 (via (at 124 100.5) (size 0.7) (drill 0.4) (layers F.Cu B.Cu) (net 1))
 (via (at 125 100.5) (size 0.7) (drill 0.4) (layers F.Cu B.Cu) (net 1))
 (via (at 126 100.5) (size 0.7) (drill 0.4) (layers F.Cu B.Cu) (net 1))
 (via (at 127 100.5) (size 0.7) (drill 0.4) (layers F.Cu B.Cu) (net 1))
 (via (at 128 100.5) (size 0.7) (drill 0.4) (layers F.Cu B.Cu) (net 1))
 (via (at 131.5 104) (size 0.7) (drill 0.4) (layers F.Cu B.Cu) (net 1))
 (via (at 131.5 114) (size 0.7) (drill 0.4) (layers F.Cu B.Cu) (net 1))
 (via (at 100.5 105) (size 0.7) (drill 0.4) (layers F.Cu B.Cu) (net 1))
 (via (at 100.5 113) (size 0.7) (drill 0.4) (layers F.Cu B.Cu) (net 1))
 (via (at 131.5 113) (size 0.7) (drill 0.4) (layers F.Cu B.Cu) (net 1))
 (via (at 131.5 105) (size 0.7) (drill 0.4) (layers F.Cu B.Cu) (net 1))
 (segment (start 129.9954 108.9954) (end 130 109) (width 1) (layer F.Cu) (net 3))
 (segment (start 117.3768 109) (end 117.3646 108.9878) (width 1) (layer F.Cu) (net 3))
 (segment (start 130 109) (end 117.3768 109) (width 1) (layer F.Cu) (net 3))
 (segment (start 102.0442 108.9878) (end 102.032 109) (width 1) (layer F.Cu) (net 2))
 (segment (start 115.2146 108.9878) (end 102.0442 108.9878) (width 1) (layer F.Cu) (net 2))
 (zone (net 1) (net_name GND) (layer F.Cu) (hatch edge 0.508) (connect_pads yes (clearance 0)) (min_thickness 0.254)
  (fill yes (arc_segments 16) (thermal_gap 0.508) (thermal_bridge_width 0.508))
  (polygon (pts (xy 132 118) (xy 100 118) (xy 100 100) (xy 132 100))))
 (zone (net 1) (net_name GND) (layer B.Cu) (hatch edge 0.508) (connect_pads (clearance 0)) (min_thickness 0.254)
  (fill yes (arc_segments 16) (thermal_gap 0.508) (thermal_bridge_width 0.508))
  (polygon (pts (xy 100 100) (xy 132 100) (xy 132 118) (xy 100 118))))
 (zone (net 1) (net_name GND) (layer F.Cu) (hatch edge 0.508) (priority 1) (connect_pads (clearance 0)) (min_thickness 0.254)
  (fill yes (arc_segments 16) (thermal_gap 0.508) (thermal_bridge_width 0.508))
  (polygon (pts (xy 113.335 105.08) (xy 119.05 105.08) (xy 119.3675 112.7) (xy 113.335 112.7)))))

